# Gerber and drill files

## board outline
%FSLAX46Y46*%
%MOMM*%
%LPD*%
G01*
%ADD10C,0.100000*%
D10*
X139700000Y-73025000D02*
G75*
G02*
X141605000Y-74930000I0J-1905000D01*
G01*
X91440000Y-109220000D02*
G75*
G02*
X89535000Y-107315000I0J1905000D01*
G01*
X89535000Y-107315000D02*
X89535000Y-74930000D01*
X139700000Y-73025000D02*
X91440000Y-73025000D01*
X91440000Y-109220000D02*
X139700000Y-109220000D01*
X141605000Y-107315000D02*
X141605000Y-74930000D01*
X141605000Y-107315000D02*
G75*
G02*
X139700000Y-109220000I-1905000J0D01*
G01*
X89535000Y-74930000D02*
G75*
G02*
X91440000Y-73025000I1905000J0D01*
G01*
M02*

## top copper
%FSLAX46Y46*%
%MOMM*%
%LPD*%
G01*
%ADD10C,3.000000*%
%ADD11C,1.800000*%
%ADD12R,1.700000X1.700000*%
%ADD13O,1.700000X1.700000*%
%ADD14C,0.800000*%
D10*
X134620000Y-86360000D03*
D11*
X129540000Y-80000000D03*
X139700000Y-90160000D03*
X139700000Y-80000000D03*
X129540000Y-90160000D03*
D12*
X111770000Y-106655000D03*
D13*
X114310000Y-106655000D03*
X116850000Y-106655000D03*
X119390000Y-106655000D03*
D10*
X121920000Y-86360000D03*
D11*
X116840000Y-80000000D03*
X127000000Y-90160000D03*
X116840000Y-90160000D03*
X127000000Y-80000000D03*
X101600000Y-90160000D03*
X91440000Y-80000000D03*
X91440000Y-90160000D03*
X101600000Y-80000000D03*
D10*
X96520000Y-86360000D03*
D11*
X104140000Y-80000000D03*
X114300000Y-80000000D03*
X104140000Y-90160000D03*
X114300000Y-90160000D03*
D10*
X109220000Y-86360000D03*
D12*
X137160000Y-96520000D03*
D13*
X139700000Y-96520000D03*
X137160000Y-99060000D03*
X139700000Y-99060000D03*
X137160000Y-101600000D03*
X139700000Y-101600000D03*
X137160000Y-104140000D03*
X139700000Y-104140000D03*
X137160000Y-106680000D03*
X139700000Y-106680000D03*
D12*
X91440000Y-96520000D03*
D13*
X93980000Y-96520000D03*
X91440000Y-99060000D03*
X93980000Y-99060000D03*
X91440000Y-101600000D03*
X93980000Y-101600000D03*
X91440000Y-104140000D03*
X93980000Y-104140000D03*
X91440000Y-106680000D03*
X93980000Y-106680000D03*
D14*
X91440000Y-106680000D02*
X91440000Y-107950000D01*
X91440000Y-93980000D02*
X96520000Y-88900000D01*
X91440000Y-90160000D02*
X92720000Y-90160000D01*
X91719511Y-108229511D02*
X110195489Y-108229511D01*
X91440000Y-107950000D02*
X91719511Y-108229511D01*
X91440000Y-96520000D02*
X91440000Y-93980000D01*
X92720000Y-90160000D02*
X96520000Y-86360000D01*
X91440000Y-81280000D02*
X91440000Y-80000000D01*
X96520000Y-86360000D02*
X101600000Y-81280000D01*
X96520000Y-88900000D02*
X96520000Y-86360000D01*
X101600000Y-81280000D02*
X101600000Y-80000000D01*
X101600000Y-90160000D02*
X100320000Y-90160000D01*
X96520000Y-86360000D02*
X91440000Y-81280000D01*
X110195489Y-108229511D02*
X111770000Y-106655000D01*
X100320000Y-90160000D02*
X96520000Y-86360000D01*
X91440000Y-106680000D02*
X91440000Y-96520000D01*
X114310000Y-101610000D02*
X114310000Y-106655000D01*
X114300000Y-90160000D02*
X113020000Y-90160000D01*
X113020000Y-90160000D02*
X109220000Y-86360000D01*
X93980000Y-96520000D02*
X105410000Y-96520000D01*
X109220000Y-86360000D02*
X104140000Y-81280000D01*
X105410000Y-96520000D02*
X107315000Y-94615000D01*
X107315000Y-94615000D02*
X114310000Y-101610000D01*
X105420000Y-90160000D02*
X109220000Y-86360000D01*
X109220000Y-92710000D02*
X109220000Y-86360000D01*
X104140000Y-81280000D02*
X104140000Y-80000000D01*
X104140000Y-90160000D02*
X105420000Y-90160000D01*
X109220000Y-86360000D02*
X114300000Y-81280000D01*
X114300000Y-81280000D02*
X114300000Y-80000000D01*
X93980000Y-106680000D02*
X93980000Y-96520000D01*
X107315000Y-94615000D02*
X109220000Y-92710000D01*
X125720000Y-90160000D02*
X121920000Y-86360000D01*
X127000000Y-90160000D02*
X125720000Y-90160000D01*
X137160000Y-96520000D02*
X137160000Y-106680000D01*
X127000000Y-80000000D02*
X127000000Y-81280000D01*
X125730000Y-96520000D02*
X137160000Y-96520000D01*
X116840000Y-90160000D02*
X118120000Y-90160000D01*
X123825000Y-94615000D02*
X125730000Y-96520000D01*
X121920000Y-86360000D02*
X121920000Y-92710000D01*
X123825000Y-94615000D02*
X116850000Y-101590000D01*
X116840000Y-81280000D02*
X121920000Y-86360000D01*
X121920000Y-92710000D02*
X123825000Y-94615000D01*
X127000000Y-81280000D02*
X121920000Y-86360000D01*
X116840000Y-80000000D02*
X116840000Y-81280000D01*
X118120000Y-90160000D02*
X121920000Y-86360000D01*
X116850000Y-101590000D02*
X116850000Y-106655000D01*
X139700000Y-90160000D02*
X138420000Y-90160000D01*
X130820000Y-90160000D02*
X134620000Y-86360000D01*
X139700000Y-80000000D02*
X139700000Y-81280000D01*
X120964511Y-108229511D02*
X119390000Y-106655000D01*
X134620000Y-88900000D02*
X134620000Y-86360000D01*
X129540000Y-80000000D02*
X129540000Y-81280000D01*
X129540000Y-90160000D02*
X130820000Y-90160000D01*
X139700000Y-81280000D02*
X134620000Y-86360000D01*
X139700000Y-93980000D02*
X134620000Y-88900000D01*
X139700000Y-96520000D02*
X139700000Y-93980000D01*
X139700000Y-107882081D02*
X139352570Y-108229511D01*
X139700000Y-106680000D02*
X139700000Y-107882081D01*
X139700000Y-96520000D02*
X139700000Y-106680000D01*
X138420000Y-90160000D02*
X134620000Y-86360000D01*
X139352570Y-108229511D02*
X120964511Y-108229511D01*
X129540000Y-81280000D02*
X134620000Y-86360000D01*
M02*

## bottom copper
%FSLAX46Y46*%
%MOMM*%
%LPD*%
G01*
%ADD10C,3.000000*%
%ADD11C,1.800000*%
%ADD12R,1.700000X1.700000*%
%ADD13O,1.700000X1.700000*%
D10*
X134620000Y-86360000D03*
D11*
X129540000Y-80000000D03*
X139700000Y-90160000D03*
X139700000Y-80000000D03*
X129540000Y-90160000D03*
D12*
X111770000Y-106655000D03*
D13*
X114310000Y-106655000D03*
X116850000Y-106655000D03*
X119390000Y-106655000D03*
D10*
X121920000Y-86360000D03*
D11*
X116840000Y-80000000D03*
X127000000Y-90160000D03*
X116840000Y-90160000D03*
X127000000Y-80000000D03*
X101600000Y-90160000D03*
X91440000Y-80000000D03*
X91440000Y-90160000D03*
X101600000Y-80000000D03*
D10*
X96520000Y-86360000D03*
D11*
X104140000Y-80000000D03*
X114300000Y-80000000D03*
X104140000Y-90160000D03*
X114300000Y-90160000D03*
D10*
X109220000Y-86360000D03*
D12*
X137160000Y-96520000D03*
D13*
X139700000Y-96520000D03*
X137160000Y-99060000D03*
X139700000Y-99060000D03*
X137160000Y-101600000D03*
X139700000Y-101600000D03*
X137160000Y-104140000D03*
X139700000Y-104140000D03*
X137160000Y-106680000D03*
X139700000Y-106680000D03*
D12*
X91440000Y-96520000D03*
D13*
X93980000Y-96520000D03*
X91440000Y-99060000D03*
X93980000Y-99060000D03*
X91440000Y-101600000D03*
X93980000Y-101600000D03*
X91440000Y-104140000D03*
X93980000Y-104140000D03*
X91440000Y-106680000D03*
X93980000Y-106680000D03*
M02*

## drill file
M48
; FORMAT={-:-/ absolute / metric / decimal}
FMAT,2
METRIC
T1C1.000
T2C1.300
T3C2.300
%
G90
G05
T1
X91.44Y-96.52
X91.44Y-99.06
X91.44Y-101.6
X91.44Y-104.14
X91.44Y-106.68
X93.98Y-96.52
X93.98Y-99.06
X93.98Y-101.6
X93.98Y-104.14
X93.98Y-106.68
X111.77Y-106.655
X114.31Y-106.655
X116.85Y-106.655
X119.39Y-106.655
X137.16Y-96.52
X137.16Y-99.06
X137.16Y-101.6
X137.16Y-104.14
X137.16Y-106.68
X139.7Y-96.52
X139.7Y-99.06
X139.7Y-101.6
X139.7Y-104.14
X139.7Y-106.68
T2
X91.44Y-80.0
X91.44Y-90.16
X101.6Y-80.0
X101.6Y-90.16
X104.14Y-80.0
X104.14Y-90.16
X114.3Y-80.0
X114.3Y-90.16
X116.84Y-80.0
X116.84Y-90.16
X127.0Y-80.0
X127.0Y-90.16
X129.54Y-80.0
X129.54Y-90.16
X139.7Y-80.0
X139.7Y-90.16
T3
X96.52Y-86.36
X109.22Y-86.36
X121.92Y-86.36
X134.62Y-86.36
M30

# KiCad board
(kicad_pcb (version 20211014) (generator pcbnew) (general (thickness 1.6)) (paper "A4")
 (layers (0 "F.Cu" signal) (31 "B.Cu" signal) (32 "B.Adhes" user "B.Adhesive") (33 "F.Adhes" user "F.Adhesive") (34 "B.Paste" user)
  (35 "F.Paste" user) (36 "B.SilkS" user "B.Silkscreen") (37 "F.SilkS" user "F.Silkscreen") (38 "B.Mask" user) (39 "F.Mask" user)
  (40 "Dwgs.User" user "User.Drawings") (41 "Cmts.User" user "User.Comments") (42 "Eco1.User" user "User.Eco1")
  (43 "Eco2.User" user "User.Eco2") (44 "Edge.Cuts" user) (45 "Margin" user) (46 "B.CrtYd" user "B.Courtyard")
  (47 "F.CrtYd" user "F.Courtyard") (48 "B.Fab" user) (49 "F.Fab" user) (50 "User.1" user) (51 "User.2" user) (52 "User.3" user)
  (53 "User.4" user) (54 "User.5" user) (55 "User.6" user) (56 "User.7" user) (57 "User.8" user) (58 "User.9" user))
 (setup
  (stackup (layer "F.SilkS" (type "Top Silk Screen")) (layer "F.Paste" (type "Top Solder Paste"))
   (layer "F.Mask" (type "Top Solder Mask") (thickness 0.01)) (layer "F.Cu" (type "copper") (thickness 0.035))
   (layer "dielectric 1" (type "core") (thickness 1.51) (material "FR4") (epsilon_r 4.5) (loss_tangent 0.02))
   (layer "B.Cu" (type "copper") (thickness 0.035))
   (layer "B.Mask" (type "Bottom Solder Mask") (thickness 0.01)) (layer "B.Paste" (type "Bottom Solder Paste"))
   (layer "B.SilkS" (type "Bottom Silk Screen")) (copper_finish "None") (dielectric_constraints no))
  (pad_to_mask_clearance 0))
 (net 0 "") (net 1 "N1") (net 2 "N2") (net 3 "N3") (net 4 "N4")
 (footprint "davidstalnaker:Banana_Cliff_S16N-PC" (layer "F.Cu") (at 134.62 86.36)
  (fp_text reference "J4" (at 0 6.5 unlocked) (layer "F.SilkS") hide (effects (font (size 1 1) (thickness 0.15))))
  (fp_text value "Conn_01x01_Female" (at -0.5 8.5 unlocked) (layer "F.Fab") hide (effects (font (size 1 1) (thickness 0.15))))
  (pad "1" thru_hole circle (at 0 0) (size 3 3) (drill 2.3) (layers *.Cu *.Mask) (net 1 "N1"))
  (pad "1" thru_hole circle (at -5.08 -6.36) (size 1.8 1.8) (drill 1.3) (layers *.Cu *.Mask) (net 1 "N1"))
  (pad "1" thru_hole circle (at 5.08 3.8) (size 1.8 1.8) (drill 1.3) (layers *.Cu *.Mask) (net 1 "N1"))
  (pad "1" thru_hole circle (at 5.08 -6.36) (size 1.8 1.8) (drill 1.3) (layers *.Cu *.Mask) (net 1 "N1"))
  (pad "1" thru_hole circle (at -5.08 3.8) (size 1.8 1.8) (drill 1.3) (layers *.Cu *.Mask) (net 1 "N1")))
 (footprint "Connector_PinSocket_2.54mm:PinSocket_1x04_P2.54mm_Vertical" (layer "F.Cu") (at 111.77 106.655 90)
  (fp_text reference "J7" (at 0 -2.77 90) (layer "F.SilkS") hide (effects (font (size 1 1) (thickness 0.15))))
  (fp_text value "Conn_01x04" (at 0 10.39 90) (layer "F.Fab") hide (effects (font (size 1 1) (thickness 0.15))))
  (pad "1" thru_hole rect locked (at 0 0 90) (size 1.7 1.7) (drill 1) (layers *.Cu *.Mask) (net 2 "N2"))
  (pad "2" thru_hole oval locked (at 0 2.54 90) (size 1.7 1.7) (drill 1) (layers *.Cu *.Mask) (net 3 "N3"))
  (pad "3" thru_hole oval locked (at 0 5.08 90) (size 1.7 1.7) (drill 1) (layers *.Cu *.Mask) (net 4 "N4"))
  (pad "4" thru_hole oval locked (at 0 7.62 90) (size 1.7 1.7) (drill 1) (layers *.Cu *.Mask) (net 1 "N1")))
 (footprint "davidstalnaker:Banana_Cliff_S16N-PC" (layer "F.Cu") (at 121.92 86.36)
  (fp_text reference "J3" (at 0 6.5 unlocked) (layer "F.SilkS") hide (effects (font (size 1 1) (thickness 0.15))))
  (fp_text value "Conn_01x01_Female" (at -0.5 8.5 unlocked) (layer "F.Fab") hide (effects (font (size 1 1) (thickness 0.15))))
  (pad "1" thru_hole circle (at 0 0) (size 3 3) (drill 2.3) (layers *.Cu *.Mask) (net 4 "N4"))
  (pad "1" thru_hole circle (at -5.08 -6.36) (size 1.8 1.8) (drill 1.3) (layers *.Cu *.Mask) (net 4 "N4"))
  (pad "1" thru_hole circle (at 5.08 3.8) (size 1.8 1.8) (drill 1.3) (layers *.Cu *.Mask) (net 4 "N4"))
  (pad "1" thru_hole circle (at -5.08 3.8) (size 1.8 1.8) (drill 1.3) (layers *.Cu *.Mask) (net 4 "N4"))
  (pad "1" thru_hole circle (at 5.08 -6.36) (size 1.8 1.8) (drill 1.3) (layers *.Cu *.Mask) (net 4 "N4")))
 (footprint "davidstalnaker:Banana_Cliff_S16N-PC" (layer "F.Cu") (at 96.52 86.36)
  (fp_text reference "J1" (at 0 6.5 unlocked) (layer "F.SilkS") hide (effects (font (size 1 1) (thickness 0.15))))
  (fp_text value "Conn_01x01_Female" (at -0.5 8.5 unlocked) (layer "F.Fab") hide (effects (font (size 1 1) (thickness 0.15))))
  (pad "1" thru_hole circle (at 5.08 3.8) (size 1.8 1.8) (drill 1.3) (layers *.Cu *.Mask) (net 2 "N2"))
  (pad "1" thru_hole circle (at -5.08 -6.36) (size 1.8 1.8) (drill 1.3) (layers *.Cu *.Mask) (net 2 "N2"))
  (pad "1" thru_hole circle (at -5.08 3.8) (size 1.8 1.8) (drill 1.3) (layers *.Cu *.Mask) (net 2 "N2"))
  (pad "1" thru_hole circle (at 5.08 -6.36) (size 1.8 1.8) (drill 1.3) (layers *.Cu *.Mask) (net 2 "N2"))
  (pad "1" thru_hole circle (at 0 0) (size 3 3) (drill 2.3) (layers *.Cu *.Mask) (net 2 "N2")))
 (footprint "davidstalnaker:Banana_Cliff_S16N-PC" (layer "F.Cu") (at 109.22 86.36)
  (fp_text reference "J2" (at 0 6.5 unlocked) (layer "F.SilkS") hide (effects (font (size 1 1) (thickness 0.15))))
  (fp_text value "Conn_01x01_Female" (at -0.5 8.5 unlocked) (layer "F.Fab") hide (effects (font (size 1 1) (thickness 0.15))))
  (pad "1" thru_hole circle (at -5.08 -6.36) (size 1.8 1.8) (drill 1.3) (layers *.Cu *.Mask) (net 3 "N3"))
  (pad "1" thru_hole circle (at 5.08 -6.36) (size 1.8 1.8) (drill 1.3) (layers *.Cu *.Mask) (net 3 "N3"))
  (pad "1" thru_hole circle (at -5.08 3.8) (size 1.8 1.8) (drill 1.3) (layers *.Cu *.Mask) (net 3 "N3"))
  (pad "1" thru_hole circle (at 5.08 3.8) (size 1.8 1.8) (drill 1.3) (layers *.Cu *.Mask) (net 3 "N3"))
  (pad "1" thru_hole circle (at 0 0) (size 3 3) (drill 2.3) (layers *.Cu *.Mask) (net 3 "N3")))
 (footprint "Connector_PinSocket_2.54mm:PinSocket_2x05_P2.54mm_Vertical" (layer "B.Cu") (at 137.16 96.52 180)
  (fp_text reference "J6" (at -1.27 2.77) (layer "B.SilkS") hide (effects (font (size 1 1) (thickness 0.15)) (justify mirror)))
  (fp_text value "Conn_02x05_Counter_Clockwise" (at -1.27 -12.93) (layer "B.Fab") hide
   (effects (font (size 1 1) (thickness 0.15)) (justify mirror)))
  (pad "1" thru_hole rect locked (at 0 0 180) (size 1.7 1.7) (drill 1) (layers *.Cu *.Mask) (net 4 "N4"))
  (pad "2" thru_hole oval locked (at -2.54 0 180) (size 1.7 1.7) (drill 1) (layers *.Cu *.Mask) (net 1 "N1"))
  (pad "3" thru_hole oval locked (at 0 -2.54 180) (size 1.7 1.7) (drill 1) (layers *.Cu *.Mask) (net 4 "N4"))
  (pad "4" thru_hole oval locked (at -2.54 -2.54 180) (size 1.7 1.7) (drill 1) (layers *.Cu *.Mask) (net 1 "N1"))
  (pad "5" thru_hole oval locked (at 0 -5.08 180) (size 1.7 1.7) (drill 1) (layers *.Cu *.Mask) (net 4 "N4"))
  (pad "6" thru_hole oval locked (at -2.54 -5.08 180) (size 1.7 1.7) (drill 1) (layers *.Cu *.Mask) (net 1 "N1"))
  (pad "7" thru_hole oval locked (at 0 -7.62 180) (size 1.7 1.7) (drill 1) (layers *.Cu *.Mask) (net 4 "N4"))
  (pad "8" thru_hole oval locked (at -2.54 -7.62 180) (size 1.7 1.7) (drill 1) (layers *.Cu *.Mask) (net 1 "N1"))
  (pad "9" thru_hole oval locked (at 0 -10.16 180) (size 1.7 1.7) (drill 1) (layers *.Cu *.Mask) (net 4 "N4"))
  (pad "10" thru_hole oval locked (at -2.54 -10.16 180) (size 1.7 1.7) (drill 1) (layers *.Cu *.Mask) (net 1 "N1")))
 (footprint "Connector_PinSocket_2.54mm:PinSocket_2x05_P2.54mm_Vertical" (layer "B.Cu") (at 91.44 96.52 180)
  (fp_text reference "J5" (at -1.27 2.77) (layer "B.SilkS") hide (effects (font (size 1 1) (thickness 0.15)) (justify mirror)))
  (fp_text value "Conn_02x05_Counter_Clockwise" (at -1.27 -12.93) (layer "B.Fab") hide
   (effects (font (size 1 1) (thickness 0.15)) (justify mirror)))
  (pad "1" thru_hole rect locked (at 0 0 180) (size 1.7 1.7) (drill 1) (layers *.Cu *.Mask) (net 2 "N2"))
  (pad "2" thru_hole oval locked (at -2.54 0 180) (size 1.7 1.7) (drill 1) (layers *.Cu *.Mask) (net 3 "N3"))
  (pad "3" thru_hole oval locked (at 0 -2.54 180) (size 1.7 1.7) (drill 1) (layers *.Cu *.Mask) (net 2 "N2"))
  (pad "4" thru_hole oval locked (at -2.54 -2.54 180) (size 1.7 1.7) (drill 1) (layers *.Cu *.Mask) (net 3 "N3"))
  (pad "5" thru_hole oval locked (at 0 -5.08 180) (size 1.7 1.7) (drill 1) (layers *.Cu *.Mask) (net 2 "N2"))
  (pad "6" thru_hole oval locked (at -2.54 -5.08 180) (size 1.7 1.7) (drill 1) (layers *.Cu *.Mask) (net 3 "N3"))
  (pad "7" thru_hole oval locked (at 0 -7.62 180) (size 1.7 1.7) (drill 1) (layers *.Cu *.Mask) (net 2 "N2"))
  (pad "8" thru_hole oval locked (at -2.54 -7.62 180) (size 1.7 1.7) (drill 1) (layers *.Cu *.Mask) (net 3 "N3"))
  (pad "9" thru_hole oval locked (at 0 -10.16 180) (size 1.7 1.7) (drill 1) (layers *.Cu *.Mask) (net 2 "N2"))
  (pad "10" thru_hole oval locked (at -2.54 -10.16 180) (size 1.7 1.7) (drill 1) (layers *.Cu *.Mask) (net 3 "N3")))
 (gr_arc (start 139.7 73.025) (mid 141.047038 73.582962) (end 141.605 74.93) (layer "Edge.Cuts") (width 0.1))
 (gr_arc (start 91.44 109.22) (mid 90.092962 108.662038) (end 89.535 107.315) (layer "Edge.Cuts") (width 0.1))
 (gr_line (start 89.535 107.315) (end 89.535 74.93) (layer "Edge.Cuts") (width 0.1))
 (gr_line (start 139.7 73.025) (end 91.44 73.025) (layer "Edge.Cuts") (width 0.1))
 (gr_line (start 91.44 109.22) (end 139.7 109.22) (layer "Edge.Cuts") (width 0.1))
 (gr_line (start 141.605 107.315) (end 141.605 74.93) (layer "Edge.Cuts") (width 0.1))
 (gr_arc (start 141.605 107.315) (mid 141.047038 108.662038) (end 139.7 109.22) (layer "Edge.Cuts") (width 0.1))
 (gr_arc (start 89.535 74.93) (mid 90.092962 73.582962) (end 91.44 73.025) (layer "Edge.Cuts") (width 0.1))
 (segment (start 91.44 106.68) (end 91.44 107.95) (width 0.8) (layer "F.Cu") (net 2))
 (segment (start 91.44 93.98) (end 96.52 88.9) (width 0.8) (layer "F.Cu") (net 2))
 (segment (start 91.44 90.16) (end 92.72 90.16) (width 0.8) (layer "F.Cu") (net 2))
 (segment (start 91.719511 108.229511) (end 110.195489 108.229511) (width 0.8) (layer "F.Cu") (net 2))
 (segment (start 91.44 107.95) (end 91.719511 108.229511) (width 0.8) (layer "F.Cu") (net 2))
 (segment (start 91.44 96.52) (end 91.44 93.98) (width 0.8) (layer "F.Cu") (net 2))
 (segment (start 92.72 90.16) (end 96.52 86.36) (width 0.8) (layer "F.Cu") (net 2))
 (segment (start 91.44 81.28) (end 91.44 80) (width 0.8) (layer "F.Cu") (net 2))
 (segment (start 96.52 86.36) (end 101.6 81.28) (width 0.8) (layer "F.Cu") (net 2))
 (segment (start 96.52 88.9) (end 96.52 86.36) (width 0.8) (layer "F.Cu") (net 2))
 (segment (start 101.6 81.28) (end 101.6 80) (width 0.8) (layer "F.Cu") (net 2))
 (segment (start 101.6 90.16) (end 100.32 90.16) (width 0.8) (layer "F.Cu") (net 2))
 (segment (start 96.52 86.36) (end 91.44 81.28) (width 0.8) (layer "F.Cu") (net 2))
 (segment (start 110.195489 108.229511) (end 111.77 106.655) (width 0.8) (layer "F.Cu") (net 2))
 (segment (start 100.32 90.16) (end 96.52 86.36) (width 0.8) (layer "F.Cu") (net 2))
 (segment (start 91.44 106.68) (end 91.44 96.52) (width 0.8) (layer "F.Cu") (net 2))
 (segment (start 114.31 101.61) (end 114.31 106.655) (width 0.8) (layer "F.Cu") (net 3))
 (segment (start 114.3 90.16) (end 113.02 90.16) (width 0.8) (layer "F.Cu") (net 3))
 (segment (start 113.02 90.16) (end 109.22 86.36) (width 0.8) (layer "F.Cu") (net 3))
 (segment (start 93.98 96.52) (end 105.41 96.52) (width 0.8) (layer "F.Cu") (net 3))
 (segment (start 109.22 86.36) (end 104.14 81.28) (width 0.8) (layer "F.Cu") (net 3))
 (segment (start 105.41 96.52) (end 107.315 94.615) (width 0.8) (layer "F.Cu") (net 3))
 (segment (start 107.315 94.615) (end 114.31 101.61) (width 0.8) (layer "F.Cu") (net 3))
 (segment (start 105.42 90.16) (end 109.22 86.36) (width 0.8) (layer "F.Cu") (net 3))
 (segment (start 109.22 92.71) (end 109.22 86.36) (width 0.8) (layer "F.Cu") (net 3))
 (segment (start 104.14 81.28) (end 104.14 80) (width 0.8) (layer "F.Cu") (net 3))
 (segment (start 104.14 90.16) (end 105.42 90.16) (width 0.8) (layer "F.Cu") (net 3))
 (segment (start 109.22 86.36) (end 114.3 81.28) (width 0.8) (layer "F.Cu") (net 3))
 (segment (start 114.3 81.28) (end 114.3 80) (width 0.8) (layer "F.Cu") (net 3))
 (segment (start 93.98 106.68) (end 93.98 96.52) (width 0.8) (layer "F.Cu") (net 3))
 (segment (start 107.315 94.615) (end 109.22 92.71) (width 0.8) (layer "F.Cu") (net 3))
 (segment (start 125.72 90.16) (end 121.92 86.36) (width 0.8) (layer "F.Cu") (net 4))
 (segment (start 127 90.16) (end 125.72 90.16) (width 0.8) (layer "F.Cu") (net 4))
 (segment (start 137.16 96.52) (end 137.16 106.68) (width 0.8) (layer "F.Cu") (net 4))
 (segment (start 127 80) (end 127 81.28) (width 0.8) (layer "F.Cu") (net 4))
 (segment (start 125.73 96.52) (end 137.16 96.52) (width 0.8) (layer "F.Cu") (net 4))
 (segment (start 116.84 90.16) (end 118.12 90.16) (width 0.8) (layer "F.Cu") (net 4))
 (segment (start 123.825 94.615) (end 125.73 96.52) (width 0.8) (layer "F.Cu") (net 4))
 (segment (start 121.92 86.36) (end 121.92 92.71) (width 0.8) (layer "F.Cu") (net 4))
 (segment (start 123.825 94.615) (end 116.85 101.59) (width 0.8) (layer "F.Cu") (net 4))
 (segment (start 116.84 81.28) (end 121.92 86.36) (width 0.8) (layer "F.Cu") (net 4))
 (segment (start 121.92 92.71) (end 123.825 94.615) (width 0.8) (layer "F.Cu") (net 4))
 (segment (start 127 81.28) (end 121.92 86.36) (width 0.8) (layer "F.Cu") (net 4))
 (segment (start 116.84 80) (end 116.84 81.28) (width 0.8) (layer "F.Cu") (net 4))
 (segment (start 118.12 90.16) (end 121.92 86.36) (width 0.8) (layer "F.Cu") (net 4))
 (segment (start 116.85 101.59) (end 116.85 106.655) (width 0.8) (layer "F.Cu") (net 4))
 (segment (start 139.7 90.16) (end 138.42 90.16) (width 0.8) (layer "F.Cu") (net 1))
 (segment (start 130.82 90.16) (end 134.62 86.36) (width 0.8) (layer "F.Cu") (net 1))
 (segment (start 139.7 80) (end 139.7 81.28) (width 0.8) (layer "F.Cu") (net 1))
 (segment (start 120.964511 108.229511) (end 119.39 106.655) (width 0.8) (layer "F.Cu") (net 1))
 (segment (start 134.62 88.9) (end 134.62 86.36) (width 0.8) (layer "F.Cu") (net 1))
 (segment (start 129.54 80) (end 129.54 81.28) (width 0.8) (layer "F.Cu") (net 1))
 (segment (start 129.54 90.16) (end 130.82 90.16) (width 0.8) (layer "F.Cu") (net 1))
 (segment (start 139.7 81.28) (end 134.62 86.36) (width 0.8) (layer "F.Cu") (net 1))
 (segment (start 139.7 93.98) (end 134.62 88.9) (width 0.8) (layer "F.Cu") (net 1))
 (segment (start 139.7 96.52) (end 139.7 93.98) (width 0.8) (layer "F.Cu") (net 1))
 (segment (start 139.7 107.882081) (end 139.35257 108.229511) (width 0.8) (layer "F.Cu") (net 1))
 (segment (start 139.7 106.68) (end 139.7 107.882081) (width 0.8) (layer "F.Cu") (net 1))
 (segment (start 139.7 96.52) (end 139.7 106.68) (width 0.8) (layer "F.Cu") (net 1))
 (segment (start 138.42 90.16) (end 134.62 86.36) (width 0.8) (layer "F.Cu") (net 1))
 (segment (start 139.35257 108.229511) (end 120.964511 108.229511) (width 0.8) (layer "F.Cu") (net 1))
 (segment (start 129.54 81.28) (end 134.62 86.36) (width 0.8) (layer "F.Cu") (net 1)))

